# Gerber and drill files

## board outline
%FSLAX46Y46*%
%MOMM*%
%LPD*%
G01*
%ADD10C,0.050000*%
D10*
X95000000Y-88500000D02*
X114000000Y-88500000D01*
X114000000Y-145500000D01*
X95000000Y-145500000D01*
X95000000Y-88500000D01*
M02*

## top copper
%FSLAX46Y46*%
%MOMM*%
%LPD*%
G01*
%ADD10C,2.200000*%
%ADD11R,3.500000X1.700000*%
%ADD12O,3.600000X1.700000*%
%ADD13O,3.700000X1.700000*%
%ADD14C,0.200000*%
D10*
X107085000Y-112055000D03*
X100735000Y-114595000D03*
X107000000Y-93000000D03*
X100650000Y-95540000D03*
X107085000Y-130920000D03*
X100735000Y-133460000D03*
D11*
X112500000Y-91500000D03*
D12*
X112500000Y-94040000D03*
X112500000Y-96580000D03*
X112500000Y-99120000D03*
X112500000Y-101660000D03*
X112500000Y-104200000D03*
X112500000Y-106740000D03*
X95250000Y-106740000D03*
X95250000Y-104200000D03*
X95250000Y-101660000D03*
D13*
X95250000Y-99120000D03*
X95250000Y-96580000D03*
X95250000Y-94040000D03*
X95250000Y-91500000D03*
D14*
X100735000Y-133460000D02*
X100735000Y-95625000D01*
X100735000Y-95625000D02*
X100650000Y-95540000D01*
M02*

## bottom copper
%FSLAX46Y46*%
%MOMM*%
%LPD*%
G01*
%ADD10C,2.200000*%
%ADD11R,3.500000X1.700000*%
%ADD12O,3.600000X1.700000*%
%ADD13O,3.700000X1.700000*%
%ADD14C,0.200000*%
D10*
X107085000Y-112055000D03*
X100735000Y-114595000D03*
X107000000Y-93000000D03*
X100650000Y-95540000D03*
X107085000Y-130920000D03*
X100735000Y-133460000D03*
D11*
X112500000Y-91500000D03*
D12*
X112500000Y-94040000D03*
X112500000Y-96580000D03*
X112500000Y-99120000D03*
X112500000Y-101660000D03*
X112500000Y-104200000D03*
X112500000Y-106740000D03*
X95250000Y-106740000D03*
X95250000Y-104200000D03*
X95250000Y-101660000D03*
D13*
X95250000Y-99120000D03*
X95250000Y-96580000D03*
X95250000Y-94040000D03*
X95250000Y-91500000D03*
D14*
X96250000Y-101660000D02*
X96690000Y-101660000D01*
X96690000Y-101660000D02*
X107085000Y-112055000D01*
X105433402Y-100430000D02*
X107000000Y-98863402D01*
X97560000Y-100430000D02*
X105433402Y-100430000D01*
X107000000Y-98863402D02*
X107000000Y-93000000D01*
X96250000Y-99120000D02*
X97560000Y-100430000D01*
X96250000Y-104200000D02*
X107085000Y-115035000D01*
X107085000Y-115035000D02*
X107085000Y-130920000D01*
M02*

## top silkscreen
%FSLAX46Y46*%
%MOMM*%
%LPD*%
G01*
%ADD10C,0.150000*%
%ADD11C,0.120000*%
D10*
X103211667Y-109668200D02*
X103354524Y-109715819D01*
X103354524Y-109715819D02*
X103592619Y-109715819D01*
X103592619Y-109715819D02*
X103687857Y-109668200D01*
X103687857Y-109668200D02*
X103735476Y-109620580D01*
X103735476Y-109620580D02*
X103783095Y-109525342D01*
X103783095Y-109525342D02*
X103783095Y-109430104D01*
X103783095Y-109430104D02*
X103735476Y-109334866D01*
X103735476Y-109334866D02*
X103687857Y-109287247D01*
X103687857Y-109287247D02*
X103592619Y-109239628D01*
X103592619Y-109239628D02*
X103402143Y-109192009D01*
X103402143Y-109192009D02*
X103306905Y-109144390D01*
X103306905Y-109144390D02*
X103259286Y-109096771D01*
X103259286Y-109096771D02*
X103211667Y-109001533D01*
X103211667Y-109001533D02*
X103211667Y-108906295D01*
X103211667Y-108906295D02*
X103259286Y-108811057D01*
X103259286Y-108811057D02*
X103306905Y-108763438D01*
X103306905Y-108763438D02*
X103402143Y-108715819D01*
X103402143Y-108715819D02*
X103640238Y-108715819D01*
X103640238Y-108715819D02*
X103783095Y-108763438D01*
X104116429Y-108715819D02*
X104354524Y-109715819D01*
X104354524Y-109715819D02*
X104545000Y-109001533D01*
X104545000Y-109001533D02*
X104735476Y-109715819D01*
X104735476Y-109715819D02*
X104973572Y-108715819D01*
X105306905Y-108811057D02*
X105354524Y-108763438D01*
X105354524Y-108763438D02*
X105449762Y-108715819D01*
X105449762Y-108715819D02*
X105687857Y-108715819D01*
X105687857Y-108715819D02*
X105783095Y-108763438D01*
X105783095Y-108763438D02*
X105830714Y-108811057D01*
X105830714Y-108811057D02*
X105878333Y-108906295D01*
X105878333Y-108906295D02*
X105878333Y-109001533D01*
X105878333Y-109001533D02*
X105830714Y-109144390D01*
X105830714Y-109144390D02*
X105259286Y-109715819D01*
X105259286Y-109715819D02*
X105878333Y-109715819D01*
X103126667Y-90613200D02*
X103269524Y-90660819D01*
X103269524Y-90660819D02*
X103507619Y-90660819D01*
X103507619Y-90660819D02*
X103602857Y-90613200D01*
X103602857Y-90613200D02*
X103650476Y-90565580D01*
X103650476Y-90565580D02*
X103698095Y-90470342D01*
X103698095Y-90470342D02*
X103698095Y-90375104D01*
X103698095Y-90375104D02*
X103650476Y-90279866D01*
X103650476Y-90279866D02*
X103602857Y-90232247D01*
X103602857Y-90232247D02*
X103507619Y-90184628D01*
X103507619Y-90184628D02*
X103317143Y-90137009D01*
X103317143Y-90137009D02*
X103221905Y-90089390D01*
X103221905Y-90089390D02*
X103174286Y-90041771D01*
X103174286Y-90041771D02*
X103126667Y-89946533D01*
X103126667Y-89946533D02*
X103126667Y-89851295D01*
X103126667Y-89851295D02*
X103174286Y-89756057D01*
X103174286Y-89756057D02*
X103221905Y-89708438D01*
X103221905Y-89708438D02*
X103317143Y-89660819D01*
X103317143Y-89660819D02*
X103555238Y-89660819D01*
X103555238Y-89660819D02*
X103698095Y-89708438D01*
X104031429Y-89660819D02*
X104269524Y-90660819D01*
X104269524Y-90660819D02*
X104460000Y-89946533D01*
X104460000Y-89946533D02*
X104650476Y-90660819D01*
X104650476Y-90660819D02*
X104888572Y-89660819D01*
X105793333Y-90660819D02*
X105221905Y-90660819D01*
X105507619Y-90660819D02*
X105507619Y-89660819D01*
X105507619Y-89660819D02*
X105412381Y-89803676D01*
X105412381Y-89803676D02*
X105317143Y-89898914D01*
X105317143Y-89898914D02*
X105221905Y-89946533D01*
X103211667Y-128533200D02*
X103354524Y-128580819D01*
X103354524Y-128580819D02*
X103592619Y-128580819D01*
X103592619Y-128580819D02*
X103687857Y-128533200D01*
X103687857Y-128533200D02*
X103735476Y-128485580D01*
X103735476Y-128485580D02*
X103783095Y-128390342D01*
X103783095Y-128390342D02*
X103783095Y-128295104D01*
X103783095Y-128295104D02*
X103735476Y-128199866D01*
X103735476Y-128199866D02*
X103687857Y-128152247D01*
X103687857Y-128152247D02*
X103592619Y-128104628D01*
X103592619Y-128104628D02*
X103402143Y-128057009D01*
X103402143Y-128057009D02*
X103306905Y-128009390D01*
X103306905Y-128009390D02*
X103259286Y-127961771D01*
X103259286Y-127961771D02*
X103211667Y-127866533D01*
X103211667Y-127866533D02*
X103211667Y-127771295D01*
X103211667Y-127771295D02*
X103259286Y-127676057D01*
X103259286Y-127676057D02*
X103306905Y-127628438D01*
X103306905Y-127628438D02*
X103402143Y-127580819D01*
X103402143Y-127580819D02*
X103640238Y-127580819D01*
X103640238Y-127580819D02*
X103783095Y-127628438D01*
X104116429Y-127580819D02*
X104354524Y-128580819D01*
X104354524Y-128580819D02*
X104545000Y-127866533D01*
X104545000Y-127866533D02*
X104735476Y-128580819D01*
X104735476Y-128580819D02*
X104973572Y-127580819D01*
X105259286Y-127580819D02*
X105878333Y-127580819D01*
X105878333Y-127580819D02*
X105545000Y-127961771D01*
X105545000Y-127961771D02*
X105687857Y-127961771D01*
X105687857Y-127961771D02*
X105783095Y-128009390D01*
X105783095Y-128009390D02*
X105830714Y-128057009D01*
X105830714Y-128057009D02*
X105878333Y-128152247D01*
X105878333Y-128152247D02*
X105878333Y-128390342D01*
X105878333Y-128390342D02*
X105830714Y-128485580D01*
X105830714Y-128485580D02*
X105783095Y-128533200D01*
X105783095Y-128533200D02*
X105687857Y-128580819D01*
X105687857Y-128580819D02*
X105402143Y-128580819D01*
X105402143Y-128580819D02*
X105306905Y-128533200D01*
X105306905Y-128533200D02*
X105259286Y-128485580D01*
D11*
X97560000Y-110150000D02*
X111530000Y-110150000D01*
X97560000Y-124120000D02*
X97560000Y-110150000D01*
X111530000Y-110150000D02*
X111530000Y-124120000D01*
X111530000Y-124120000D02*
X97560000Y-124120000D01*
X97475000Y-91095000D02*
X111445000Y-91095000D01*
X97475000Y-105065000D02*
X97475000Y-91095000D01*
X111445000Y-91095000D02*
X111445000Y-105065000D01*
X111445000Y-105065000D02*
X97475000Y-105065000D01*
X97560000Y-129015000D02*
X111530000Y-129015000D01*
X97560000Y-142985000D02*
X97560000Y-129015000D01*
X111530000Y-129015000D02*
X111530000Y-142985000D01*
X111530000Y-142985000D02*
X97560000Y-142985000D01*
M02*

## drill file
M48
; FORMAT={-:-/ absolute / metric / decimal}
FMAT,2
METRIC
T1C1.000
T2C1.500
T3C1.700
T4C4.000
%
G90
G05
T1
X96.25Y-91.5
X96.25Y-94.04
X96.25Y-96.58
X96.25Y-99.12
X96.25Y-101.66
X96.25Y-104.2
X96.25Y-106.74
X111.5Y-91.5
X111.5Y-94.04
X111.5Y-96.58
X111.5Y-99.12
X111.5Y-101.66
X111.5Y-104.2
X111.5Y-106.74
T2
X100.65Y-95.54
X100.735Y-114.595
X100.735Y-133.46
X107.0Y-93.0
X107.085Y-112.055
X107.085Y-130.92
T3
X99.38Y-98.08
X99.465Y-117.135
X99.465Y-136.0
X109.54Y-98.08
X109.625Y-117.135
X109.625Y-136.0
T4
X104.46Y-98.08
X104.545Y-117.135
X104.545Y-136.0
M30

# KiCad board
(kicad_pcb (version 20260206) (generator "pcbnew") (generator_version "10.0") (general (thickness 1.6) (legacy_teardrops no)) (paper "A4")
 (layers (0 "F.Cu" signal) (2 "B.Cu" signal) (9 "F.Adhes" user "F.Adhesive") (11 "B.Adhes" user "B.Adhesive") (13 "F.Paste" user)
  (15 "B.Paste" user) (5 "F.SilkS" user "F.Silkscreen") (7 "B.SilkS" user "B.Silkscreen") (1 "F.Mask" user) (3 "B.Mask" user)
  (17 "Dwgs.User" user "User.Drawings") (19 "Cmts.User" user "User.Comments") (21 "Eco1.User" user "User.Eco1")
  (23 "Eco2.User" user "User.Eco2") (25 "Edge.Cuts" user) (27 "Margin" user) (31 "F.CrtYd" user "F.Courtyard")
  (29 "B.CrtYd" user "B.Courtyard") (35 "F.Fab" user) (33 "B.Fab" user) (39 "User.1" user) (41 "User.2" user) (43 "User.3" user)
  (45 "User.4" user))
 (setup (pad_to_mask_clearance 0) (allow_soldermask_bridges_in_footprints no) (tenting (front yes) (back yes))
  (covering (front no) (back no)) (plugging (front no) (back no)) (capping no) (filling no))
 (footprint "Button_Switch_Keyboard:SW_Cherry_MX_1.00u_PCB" (layer "F.Cu") (at 107.085 112.055)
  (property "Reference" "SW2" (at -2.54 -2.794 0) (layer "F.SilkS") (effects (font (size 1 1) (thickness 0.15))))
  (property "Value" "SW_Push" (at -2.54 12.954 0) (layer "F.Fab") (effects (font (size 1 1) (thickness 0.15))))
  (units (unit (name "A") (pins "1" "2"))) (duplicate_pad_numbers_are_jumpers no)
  (fp_line (start -9.525 -1.905) (end 4.445 -1.905) (stroke (width 0.12) (type solid)) (layer "F.SilkS"))
  (fp_line (start -9.525 12.065) (end -9.525 -1.905) (stroke (width 0.12) (type solid)) (layer "F.SilkS"))
  (fp_line (start 4.445 -1.905) (end 4.445 12.065) (stroke (width 0.12) (type solid)) (layer "F.SilkS"))
  (fp_line (start 4.445 12.065) (end -9.525 12.065) (stroke (width 0.12) (type solid)) (layer "F.SilkS"))
  (pad "" np_thru_hole circle (at -7.62 5.08) (size 1.7 1.7) (drill 1.7) (layers "*.Cu" "*.Mask"))
  (pad "" np_thru_hole circle (at -2.54 5.08) (size 4 4) (drill 4) (layers "*.Cu" "*.Mask"))
  (pad "" np_thru_hole circle (at 2.54 5.08) (size 1.7 1.7) (drill 1.7) (layers "*.Cu" "*.Mask"))
  (pad "1" thru_hole circle (at 0 0) (size 2.2 2.2) (drill 1.5) (layers "*.Cu" "*.Mask") (remove_unused_layers no)
   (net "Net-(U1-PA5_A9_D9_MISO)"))
  (pad "2" thru_hole circle (at -6.35 2.54) (size 2.2 2.2) (drill 1.5) (layers "*.Cu" "*.Mask") (remove_unused_layers no) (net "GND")))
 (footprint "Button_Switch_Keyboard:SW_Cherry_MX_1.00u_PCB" (layer "F.Cu") (at 107 93)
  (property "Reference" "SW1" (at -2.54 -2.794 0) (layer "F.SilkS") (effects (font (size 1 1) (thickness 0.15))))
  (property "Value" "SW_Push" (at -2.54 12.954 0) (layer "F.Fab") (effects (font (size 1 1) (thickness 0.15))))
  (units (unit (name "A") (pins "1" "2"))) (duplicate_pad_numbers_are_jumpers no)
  (fp_line (start -9.525 -1.905) (end 4.445 -1.905) (stroke (width 0.12) (type solid)) (layer "F.SilkS"))
  (fp_line (start -9.525 12.065) (end -9.525 -1.905) (stroke (width 0.12) (type solid)) (layer "F.SilkS"))
  (fp_line (start 4.445 -1.905) (end 4.445 12.065) (stroke (width 0.12) (type solid)) (layer "F.SilkS"))
  (fp_line (start 4.445 12.065) (end -9.525 12.065) (stroke (width 0.12) (type solid)) (layer "F.SilkS"))
  (pad "" np_thru_hole circle (at -7.62 5.08) (size 1.7 1.7) (drill 1.7) (layers "*.Cu" "*.Mask"))
  (pad "" np_thru_hole circle (at -2.54 5.08) (size 4 4) (drill 4) (layers "*.Cu" "*.Mask"))
  (pad "" np_thru_hole circle (at 2.54 5.08) (size 1.7 1.7) (drill 1.7) (layers "*.Cu" "*.Mask"))
  (pad "1" thru_hole circle (at 0 0) (size 2.2 2.2) (drill 1.5) (layers "*.Cu" "*.Mask") (remove_unused_layers no)
   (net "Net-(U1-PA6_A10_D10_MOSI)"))
  (pad "2" thru_hole circle (at -6.35 2.54) (size 2.2 2.2) (drill 1.5) (layers "*.Cu" "*.Mask") (remove_unused_layers no) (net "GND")))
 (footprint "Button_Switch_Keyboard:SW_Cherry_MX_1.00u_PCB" (layer "F.Cu") (at 107.085 130.92)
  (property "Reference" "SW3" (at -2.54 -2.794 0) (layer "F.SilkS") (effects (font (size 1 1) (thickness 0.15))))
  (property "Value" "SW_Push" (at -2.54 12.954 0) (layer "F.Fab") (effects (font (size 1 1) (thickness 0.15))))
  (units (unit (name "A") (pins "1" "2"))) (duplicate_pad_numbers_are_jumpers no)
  (fp_line (start -9.525 -1.905) (end 4.445 -1.905) (stroke (width 0.12) (type solid)) (layer "F.SilkS"))
  (fp_line (start -9.525 12.065) (end -9.525 -1.905) (stroke (width 0.12) (type solid)) (layer "F.SilkS"))
  (fp_line (start 4.445 -1.905) (end 4.445 12.065) (stroke (width 0.12) (type solid)) (layer "F.SilkS"))
  (fp_line (start 4.445 12.065) (end -9.525 12.065) (stroke (width 0.12) (type solid)) (layer "F.SilkS"))
  (pad "" np_thru_hole circle (at -7.62 5.08) (size 1.7 1.7) (drill 1.7) (layers "*.Cu" "*.Mask"))
  (pad "" np_thru_hole circle (at -2.54 5.08) (size 4 4) (drill 4) (layers "*.Cu" "*.Mask"))
  (pad "" np_thru_hole circle (at 2.54 5.08) (size 1.7 1.7) (drill 1.7) (layers "*.Cu" "*.Mask"))
  (pad "1" thru_hole circle (at 0 0) (size 2.2 2.2) (drill 1.5) (layers "*.Cu" "*.Mask") (remove_unused_layers no)
   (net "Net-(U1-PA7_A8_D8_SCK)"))
  (pad "2" thru_hole circle (at -6.35 2.54) (size 2.2 2.2) (drill 1.5) (layers "*.Cu" "*.Mask") (remove_unused_layers no) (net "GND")))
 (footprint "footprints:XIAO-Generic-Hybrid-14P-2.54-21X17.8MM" (layer "B.Cu") (at 103.875 99.12 180)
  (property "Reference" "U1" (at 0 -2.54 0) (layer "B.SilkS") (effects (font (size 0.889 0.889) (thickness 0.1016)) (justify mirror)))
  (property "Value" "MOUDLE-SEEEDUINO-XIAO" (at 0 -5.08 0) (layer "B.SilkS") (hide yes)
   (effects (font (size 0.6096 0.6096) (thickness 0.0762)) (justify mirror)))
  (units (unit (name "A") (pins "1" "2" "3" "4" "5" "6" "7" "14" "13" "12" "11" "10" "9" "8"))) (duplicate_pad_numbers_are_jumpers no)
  (pad "1" thru_hole rect (at -7.625 7.62 180) (size 3.5 1.7) (drill 1 (offset -1 0)) (layers "*.Cu" "*.Mask") (remove_unused_layers no)
   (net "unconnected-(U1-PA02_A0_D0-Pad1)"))
  (pad "2" thru_hole oval (at -7.625 5.08 180) (size 3.6 1.7) (drill 1 (offset -1 0)) (layers "*.Cu" "*.Mask") (remove_unused_layers no)
   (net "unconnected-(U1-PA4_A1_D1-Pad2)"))
  (pad "3" thru_hole oval (at -7.625 2.54 180) (size 3.6 1.7) (drill 1 (offset -1 0)) (layers "*.Cu" "*.Mask") (remove_unused_layers no)
   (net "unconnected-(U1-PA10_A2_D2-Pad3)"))
  (pad "4" thru_hole oval (at -7.625 0 180) (size 3.6 1.7) (drill 1 (offset -1 0)) (layers "*.Cu" "*.Mask") (remove_unused_layers no)
   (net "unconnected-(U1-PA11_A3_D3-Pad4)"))
  (pad "5" thru_hole oval (at -7.625 -2.54 180) (size 3.6 1.7) (drill 1 (offset -1 0)) (layers "*.Cu" "*.Mask") (remove_unused_layers no)
   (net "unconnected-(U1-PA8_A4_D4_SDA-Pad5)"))
  (pad "6" thru_hole oval (at -7.625 -5.08) (size 3.6 1.7) (drill 1 (offset 1 0)) (layers "*.Cu" "*.Mask") (remove_unused_layers no)
   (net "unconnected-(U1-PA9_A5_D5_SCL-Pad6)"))
  (pad "7" thru_hole oval (at -7.625 -7.62 180) (size 3.6 1.7) (drill 1 (offset -1 0)) (layers "*.Cu" "*.Mask") (remove_unused_layers no)
   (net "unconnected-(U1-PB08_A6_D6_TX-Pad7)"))
  (pad "8" thru_hole oval (at 7.625 -7.62 180) (size 3.6 1.7) (drill 1 (offset 1 0)) (layers "*.Cu" "*.Mask") (remove_unused_layers no)
   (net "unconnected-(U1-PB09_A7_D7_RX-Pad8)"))
  (pad "9" thru_hole oval (at 7.625 -5.08 180) (size 3.6 1.7) (drill 1 (offset 1 0)) (layers "*.Cu" "*.Mask") (remove_unused_layers no)
   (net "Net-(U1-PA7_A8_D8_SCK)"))
  (pad "10" thru_hole oval (at 7.625 -2.54 180) (size 3.6 1.7) (drill 1 (offset 1 0)) (layers "*.Cu" "*.Mask") (remove_unused_layers no)
   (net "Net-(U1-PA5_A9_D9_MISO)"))
  (pad "11" thru_hole oval (at 7.625 0 180) (size 3.7 1.7) (drill 1 (offset 1 0)) (layers "*.Cu" "*.Mask") (remove_unused_layers no)
   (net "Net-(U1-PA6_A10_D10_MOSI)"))
  (pad "12" thru_hole oval (at 7.625 2.54 180) (size 3.7 1.7) (drill 1 (offset 1 0)) (layers "*.Cu" "*.Mask") (remove_unused_layers no)
   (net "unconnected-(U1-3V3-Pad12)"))
  (pad "13" thru_hole oval (at 7.625 5.08 180) (size 3.7 1.7) (drill 1 (offset 1 0)) (layers "*.Cu" "*.Mask") (remove_unused_layers no)
   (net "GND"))
  (pad "14" thru_hole oval (at 7.625 7.62 180) (size 3.7 1.7) (drill 1 (offset 1 0)) (layers "*.Cu" "*.Mask") (remove_unused_layers no)
   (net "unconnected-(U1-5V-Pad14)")))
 (gr_rect (start 95 88.5) (end 114 145.5) (stroke (width 0.05) (type default)) (fill no) (layer "Edge.Cuts"))
 (segment (start 96.25 101.66) (end 96.69 101.66) (width 0.2) (layer "B.Cu") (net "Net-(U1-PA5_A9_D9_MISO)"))
 (segment (start 96.69 101.66) (end 107.085 112.055) (width 0.2) (layer "B.Cu") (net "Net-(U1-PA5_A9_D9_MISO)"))
 (segment (start 100.735 133.46) (end 100.735 95.625) (width 0.2) (layer "F.Cu") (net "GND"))
 (segment (start 100.735 95.625) (end 100.65 95.54) (width 0.2) (layer "F.Cu") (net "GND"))
 (segment (start 105.433402 100.43) (end 107 98.863402) (width 0.2) (layer "B.Cu") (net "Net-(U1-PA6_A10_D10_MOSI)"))
 (segment (start 97.56 100.43) (end 105.433402 100.43) (width 0.2) (layer "B.Cu") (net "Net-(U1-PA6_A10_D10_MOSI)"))
 (segment (start 107 98.863402) (end 107 93) (width 0.2) (layer "B.Cu") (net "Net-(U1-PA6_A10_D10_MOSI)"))
 (segment (start 96.25 99.12) (end 97.56 100.43) (width 0.2) (layer "B.Cu") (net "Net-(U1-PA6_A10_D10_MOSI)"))
 (segment (start 96.25 104.2) (end 107.085 115.035) (width 0.2) (layer "B.Cu") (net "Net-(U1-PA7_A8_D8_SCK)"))
 (segment (start 107.085 115.035) (end 107.085 130.92) (width 0.2) (layer "B.Cu") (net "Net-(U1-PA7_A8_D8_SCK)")))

